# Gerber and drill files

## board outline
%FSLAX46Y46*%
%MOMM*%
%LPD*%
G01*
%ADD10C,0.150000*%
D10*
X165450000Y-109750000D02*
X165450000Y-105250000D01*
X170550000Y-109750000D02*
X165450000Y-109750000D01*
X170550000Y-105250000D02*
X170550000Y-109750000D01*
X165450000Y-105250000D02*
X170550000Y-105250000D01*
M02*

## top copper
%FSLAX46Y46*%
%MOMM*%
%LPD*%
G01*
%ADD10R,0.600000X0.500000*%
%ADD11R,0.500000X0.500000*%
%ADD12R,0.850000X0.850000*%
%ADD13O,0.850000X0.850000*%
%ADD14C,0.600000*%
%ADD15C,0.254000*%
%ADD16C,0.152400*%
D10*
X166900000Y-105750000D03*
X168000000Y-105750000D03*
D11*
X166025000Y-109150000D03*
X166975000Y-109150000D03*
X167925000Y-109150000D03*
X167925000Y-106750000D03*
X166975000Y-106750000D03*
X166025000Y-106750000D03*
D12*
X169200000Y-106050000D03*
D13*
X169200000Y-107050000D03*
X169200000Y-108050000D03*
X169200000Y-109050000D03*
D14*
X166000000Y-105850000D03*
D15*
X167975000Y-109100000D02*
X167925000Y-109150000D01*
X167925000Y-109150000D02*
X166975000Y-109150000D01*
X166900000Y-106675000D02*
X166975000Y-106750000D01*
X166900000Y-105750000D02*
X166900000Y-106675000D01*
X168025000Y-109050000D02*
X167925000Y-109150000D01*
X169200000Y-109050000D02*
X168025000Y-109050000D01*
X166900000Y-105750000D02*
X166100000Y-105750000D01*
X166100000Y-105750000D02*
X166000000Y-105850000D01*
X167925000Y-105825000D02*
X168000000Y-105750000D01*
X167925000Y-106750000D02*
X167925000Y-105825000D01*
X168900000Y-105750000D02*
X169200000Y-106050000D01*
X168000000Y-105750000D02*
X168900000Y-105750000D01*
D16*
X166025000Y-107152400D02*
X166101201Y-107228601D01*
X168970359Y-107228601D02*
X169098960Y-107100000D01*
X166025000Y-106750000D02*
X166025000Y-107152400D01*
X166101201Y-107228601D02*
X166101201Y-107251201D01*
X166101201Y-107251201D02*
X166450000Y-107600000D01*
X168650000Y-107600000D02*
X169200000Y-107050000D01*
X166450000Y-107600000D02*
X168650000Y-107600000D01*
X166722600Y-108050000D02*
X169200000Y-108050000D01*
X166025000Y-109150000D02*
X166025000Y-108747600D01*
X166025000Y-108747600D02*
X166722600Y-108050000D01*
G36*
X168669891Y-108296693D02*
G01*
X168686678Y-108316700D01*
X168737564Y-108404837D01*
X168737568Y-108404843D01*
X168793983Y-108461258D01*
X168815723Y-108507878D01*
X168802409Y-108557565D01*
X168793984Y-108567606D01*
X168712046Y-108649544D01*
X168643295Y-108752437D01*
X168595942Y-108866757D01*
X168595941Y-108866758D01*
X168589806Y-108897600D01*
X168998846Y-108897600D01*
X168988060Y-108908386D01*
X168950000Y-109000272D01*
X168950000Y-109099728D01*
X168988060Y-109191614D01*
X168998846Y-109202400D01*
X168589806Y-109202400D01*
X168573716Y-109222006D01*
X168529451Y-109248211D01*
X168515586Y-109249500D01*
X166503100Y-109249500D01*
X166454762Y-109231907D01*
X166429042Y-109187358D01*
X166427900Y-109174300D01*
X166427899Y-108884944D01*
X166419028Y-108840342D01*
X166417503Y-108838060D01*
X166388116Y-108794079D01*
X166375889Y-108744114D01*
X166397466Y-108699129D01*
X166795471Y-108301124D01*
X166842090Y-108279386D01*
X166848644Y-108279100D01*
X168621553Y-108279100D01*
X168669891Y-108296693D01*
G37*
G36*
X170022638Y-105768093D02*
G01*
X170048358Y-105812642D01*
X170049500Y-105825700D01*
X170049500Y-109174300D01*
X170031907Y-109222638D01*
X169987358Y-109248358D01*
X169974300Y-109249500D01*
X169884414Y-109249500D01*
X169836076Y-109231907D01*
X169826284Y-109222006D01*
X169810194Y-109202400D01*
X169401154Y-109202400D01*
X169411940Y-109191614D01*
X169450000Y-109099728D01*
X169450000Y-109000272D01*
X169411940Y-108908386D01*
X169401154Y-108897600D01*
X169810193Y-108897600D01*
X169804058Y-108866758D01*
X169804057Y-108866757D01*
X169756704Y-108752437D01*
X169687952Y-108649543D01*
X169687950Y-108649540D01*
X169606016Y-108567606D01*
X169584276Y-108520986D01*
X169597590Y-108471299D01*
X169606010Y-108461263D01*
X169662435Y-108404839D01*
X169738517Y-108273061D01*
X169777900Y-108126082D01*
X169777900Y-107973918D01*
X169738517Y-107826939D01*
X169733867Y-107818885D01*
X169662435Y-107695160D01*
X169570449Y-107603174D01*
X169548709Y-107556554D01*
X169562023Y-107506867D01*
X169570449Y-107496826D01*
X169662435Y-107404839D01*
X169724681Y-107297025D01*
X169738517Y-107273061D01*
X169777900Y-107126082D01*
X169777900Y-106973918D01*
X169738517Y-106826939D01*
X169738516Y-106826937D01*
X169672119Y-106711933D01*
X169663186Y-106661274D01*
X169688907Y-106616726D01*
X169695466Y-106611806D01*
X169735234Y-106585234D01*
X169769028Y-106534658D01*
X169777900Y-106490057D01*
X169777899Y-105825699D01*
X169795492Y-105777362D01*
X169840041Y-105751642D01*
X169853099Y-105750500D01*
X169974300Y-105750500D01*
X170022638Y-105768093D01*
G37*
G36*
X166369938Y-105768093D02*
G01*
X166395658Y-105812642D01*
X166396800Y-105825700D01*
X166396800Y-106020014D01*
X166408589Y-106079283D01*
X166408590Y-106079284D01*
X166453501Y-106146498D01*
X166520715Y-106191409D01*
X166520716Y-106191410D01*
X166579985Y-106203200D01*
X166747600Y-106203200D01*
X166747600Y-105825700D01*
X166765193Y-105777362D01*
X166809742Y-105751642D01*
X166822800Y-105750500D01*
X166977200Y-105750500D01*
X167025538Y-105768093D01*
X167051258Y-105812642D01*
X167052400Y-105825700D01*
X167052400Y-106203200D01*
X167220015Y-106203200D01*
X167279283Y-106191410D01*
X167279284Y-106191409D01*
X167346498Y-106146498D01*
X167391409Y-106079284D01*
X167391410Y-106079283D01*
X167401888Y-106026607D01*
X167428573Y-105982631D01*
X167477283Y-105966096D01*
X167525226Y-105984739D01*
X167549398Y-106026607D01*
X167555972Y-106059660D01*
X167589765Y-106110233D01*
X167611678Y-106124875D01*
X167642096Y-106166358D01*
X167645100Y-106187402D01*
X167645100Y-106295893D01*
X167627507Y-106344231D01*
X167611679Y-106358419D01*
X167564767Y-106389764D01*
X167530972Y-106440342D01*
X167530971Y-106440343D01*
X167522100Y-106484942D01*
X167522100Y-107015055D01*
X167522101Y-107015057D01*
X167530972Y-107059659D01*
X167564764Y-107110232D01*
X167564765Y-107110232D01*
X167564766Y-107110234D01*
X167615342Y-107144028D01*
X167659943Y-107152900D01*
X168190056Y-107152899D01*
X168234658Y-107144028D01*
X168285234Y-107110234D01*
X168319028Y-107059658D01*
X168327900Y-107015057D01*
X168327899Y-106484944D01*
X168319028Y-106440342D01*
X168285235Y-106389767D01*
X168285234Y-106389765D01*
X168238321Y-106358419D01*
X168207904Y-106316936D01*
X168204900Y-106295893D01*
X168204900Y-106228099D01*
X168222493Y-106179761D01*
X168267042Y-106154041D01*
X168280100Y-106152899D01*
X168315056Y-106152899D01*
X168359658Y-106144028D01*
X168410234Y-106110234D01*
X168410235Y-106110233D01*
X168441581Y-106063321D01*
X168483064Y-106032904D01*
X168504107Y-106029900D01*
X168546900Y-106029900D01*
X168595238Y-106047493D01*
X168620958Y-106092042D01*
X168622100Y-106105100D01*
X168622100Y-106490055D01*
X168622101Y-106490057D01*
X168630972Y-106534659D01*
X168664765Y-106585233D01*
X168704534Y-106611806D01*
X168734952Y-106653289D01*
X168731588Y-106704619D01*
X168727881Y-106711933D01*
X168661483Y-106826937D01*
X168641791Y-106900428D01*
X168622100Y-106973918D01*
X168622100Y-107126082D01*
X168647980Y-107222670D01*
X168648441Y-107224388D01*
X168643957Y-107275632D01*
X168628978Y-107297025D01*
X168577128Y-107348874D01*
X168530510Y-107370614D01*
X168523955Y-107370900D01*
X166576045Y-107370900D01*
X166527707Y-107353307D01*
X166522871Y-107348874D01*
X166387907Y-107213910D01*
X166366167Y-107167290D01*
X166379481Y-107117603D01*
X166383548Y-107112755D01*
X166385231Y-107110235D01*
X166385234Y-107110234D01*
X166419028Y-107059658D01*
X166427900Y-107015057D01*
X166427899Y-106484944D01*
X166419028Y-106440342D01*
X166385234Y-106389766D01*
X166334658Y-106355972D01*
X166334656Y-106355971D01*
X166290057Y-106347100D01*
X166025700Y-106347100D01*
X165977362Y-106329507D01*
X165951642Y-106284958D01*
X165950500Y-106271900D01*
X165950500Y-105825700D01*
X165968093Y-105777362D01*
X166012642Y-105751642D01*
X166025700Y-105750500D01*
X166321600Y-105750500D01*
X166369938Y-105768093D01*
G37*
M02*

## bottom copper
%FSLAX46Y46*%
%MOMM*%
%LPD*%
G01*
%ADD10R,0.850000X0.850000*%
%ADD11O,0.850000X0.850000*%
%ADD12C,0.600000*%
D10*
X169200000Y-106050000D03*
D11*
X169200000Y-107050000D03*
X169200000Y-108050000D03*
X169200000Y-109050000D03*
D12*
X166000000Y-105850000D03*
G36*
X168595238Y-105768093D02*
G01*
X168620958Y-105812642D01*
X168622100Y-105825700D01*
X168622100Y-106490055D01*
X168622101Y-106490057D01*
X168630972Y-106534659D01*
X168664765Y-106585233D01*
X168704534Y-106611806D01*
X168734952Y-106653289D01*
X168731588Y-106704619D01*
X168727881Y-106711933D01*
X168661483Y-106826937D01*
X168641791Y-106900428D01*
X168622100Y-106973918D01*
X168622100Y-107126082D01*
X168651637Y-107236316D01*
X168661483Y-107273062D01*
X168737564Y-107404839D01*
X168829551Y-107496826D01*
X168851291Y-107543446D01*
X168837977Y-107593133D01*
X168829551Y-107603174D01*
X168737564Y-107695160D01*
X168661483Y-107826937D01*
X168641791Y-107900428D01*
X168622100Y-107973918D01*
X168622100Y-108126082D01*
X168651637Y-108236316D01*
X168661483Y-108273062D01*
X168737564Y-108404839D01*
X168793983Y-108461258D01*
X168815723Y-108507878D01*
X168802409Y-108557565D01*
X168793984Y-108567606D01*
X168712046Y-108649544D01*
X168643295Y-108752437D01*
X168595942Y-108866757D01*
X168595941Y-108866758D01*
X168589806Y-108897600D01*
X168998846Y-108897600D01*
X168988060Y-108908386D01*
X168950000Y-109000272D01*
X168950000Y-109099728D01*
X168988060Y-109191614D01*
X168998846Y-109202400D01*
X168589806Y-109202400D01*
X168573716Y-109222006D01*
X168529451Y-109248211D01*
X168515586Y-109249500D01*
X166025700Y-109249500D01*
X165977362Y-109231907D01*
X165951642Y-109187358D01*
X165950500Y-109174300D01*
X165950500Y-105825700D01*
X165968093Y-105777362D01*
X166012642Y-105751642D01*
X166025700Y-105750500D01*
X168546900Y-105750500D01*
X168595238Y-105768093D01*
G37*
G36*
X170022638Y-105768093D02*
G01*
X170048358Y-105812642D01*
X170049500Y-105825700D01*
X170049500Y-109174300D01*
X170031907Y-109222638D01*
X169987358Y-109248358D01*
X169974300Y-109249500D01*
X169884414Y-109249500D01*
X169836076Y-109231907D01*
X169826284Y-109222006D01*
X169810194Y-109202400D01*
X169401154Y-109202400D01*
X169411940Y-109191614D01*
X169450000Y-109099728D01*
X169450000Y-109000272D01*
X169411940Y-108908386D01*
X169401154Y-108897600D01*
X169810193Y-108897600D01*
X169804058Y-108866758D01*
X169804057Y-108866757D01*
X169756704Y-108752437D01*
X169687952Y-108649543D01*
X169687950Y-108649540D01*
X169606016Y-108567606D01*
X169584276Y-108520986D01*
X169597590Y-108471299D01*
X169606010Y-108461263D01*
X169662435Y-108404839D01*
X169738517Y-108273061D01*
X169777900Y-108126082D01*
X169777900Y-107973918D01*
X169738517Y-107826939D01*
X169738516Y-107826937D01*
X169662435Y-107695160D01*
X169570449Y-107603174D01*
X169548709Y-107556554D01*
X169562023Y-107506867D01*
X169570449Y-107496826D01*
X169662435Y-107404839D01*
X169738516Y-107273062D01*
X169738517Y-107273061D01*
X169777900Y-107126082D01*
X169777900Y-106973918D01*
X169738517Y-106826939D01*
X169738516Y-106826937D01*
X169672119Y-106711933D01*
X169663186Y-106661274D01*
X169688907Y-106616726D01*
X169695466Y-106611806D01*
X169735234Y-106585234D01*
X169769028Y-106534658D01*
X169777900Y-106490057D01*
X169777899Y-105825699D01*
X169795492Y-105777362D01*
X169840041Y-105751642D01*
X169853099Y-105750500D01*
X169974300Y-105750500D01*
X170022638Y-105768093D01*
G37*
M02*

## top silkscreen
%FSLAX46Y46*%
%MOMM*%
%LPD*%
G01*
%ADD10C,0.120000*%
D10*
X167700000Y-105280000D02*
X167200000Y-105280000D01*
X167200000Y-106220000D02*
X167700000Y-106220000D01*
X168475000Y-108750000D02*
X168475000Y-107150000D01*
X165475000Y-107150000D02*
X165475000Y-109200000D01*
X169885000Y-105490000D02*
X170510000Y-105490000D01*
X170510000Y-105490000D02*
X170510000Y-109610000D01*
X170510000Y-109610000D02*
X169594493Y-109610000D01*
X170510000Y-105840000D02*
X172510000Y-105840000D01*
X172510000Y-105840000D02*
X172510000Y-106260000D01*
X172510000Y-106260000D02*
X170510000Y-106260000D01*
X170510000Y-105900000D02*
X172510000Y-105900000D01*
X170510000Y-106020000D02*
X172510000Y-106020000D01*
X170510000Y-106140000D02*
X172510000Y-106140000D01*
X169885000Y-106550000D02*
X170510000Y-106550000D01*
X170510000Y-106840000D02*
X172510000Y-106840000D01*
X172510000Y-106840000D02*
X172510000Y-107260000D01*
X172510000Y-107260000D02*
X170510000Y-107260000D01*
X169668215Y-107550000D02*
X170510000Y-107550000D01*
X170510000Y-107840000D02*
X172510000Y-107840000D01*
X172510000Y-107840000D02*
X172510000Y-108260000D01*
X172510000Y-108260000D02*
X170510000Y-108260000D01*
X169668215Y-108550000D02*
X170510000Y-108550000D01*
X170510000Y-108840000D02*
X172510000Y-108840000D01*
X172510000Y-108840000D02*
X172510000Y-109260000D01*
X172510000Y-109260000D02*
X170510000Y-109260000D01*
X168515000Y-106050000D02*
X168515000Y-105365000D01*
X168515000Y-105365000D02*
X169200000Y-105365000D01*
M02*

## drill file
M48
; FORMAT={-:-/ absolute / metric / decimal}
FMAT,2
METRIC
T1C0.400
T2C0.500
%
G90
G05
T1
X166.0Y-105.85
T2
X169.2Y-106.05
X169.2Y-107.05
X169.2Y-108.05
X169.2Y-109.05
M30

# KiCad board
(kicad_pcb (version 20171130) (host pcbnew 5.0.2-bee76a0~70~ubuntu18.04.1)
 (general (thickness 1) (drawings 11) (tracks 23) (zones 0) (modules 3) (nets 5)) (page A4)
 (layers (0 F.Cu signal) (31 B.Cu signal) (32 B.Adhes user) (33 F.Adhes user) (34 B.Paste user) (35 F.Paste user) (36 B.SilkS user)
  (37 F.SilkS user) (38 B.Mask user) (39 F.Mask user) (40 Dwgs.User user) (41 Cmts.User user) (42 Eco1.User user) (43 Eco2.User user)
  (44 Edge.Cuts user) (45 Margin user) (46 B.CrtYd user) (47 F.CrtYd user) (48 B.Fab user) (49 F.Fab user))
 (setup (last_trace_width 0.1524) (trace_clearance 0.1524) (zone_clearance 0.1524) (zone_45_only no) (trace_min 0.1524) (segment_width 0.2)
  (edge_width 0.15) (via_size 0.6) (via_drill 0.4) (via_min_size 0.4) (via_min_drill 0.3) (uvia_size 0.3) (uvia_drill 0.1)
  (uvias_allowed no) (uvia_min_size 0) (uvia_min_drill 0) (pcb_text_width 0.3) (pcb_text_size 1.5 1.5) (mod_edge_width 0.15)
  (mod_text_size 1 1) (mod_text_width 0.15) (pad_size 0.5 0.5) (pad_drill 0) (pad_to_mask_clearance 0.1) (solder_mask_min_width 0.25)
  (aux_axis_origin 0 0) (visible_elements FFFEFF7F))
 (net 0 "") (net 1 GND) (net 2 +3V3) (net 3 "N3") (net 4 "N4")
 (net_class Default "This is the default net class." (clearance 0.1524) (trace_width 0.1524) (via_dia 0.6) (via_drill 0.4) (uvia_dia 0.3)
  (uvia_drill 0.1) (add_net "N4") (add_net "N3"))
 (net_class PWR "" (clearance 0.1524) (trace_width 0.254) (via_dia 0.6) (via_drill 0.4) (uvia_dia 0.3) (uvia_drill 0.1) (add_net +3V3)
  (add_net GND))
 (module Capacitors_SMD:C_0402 (layer F.Cu) (at 167.45 105.75)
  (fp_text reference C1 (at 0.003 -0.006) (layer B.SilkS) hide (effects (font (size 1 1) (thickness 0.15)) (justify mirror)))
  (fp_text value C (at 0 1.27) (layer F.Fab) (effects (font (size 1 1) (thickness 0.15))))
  (fp_line (start 0.25 -0.47) (end -0.25 -0.47) (layer F.SilkS) (width 0.12))
  (fp_line (start -0.25 0.47) (end 0.25 0.47) (layer F.SilkS) (width 0.12))
  (pad 1 smd rect (at -0.55 0) (size 0.6 0.5) (layers F.Cu F.Paste F.Mask) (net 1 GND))
  (pad 2 smd rect (at 0.55 0) (size 0.6 0.5) (layers F.Cu F.Paste F.Mask) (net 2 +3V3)))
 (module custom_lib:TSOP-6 (layer F.Cu) (at 166.975 107.95 90)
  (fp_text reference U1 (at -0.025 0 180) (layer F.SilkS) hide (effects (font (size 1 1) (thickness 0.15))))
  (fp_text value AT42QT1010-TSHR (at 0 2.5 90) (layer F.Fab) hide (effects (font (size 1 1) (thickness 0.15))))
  (fp_line (start -0.8 1.5) (end 0.8 1.5) (layer F.SilkS) (width 0.12))
  (fp_line (start 0.8 -1.5) (end -1.25 -1.5) (layer F.SilkS) (width 0.12))
  (pad 1 smd rect (at -1.2 -0.95 90) (size 0.5 0.5) (layers F.Cu F.Paste F.Mask) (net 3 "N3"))
  (pad 2 smd rect (at -1.2 0 90) (size 0.5 0.5) (layers F.Cu F.Paste F.Mask) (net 1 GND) (zone_connect 2))
  (pad 3 smd rect (at -1.2 0.95 90) (size 0.5 0.5) (layers F.Cu F.Paste F.Mask) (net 1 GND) (zone_connect 2))
  (pad 4 smd rect (at 1.2 0.95 90) (size 0.5 0.5) (layers F.Cu F.Paste F.Mask) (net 2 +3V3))
  (pad 5 smd rect (at 1.2 0 90) (size 0.5 0.5) (layers F.Cu F.Paste F.Mask) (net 1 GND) (zone_connect 2))
  (pad 6 smd rect (at 1.2 -0.95 90) (size 0.5 0.5) (layers F.Cu F.Paste F.Mask) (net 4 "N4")))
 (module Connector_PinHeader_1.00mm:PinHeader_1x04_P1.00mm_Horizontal (layer F.Cu) (at 169.2 106.05)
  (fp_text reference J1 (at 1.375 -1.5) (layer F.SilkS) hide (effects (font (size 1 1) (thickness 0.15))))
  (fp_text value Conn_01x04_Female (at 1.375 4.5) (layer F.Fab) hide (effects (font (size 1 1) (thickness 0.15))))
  (fp_line (start 0.685 -0.56) (end 1.31 -0.56) (layer F.SilkS) (width 0.12))
  (fp_line (start 1.31 -0.56) (end 1.31 3.56) (layer F.SilkS) (width 0.12))
  (fp_line (start 1.31 3.56) (end 0.394493 3.56) (layer F.SilkS) (width 0.12))
  (fp_line (start 1.31 -0.21) (end 3.31 -0.21) (layer F.SilkS) (width 0.12))
  (fp_line (start 3.31 -0.21) (end 3.31 0.21) (layer F.SilkS) (width 0.12))
  (fp_line (start 3.31 0.21) (end 1.31 0.21) (layer F.SilkS) (width 0.12))
  (fp_line (start 1.31 -0.15) (end 3.31 -0.15) (layer F.SilkS) (width 0.12))
  (fp_line (start 1.31 -0.03) (end 3.31 -0.03) (layer F.SilkS) (width 0.12))
  (fp_line (start 1.31 0.09) (end 3.31 0.09) (layer F.SilkS) (width 0.12))
  (fp_line (start 0.685 0.5) (end 1.31 0.5) (layer F.SilkS) (width 0.12))
  (fp_line (start 1.31 0.79) (end 3.31 0.79) (layer F.SilkS) (width 0.12))
  (fp_line (start 3.31 0.79) (end 3.31 1.21) (layer F.SilkS) (width 0.12))
  (fp_line (start 3.31 1.21) (end 1.31 1.21) (layer F.SilkS) (width 0.12))
  (fp_line (start 0.468215 1.5) (end 1.31 1.5) (layer F.SilkS) (width 0.12))
  (fp_line (start 1.31 1.79) (end 3.31 1.79) (layer F.SilkS) (width 0.12))
  (fp_line (start 3.31 1.79) (end 3.31 2.21) (layer F.SilkS) (width 0.12))
  (fp_line (start 3.31 2.21) (end 1.31 2.21) (layer F.SilkS) (width 0.12))
  (fp_line (start 0.468215 2.5) (end 1.31 2.5) (layer F.SilkS) (width 0.12))
  (fp_line (start 1.31 2.79) (end 3.31 2.79) (layer F.SilkS) (width 0.12))
  (fp_line (start 3.31 2.79) (end 3.31 3.21) (layer F.SilkS) (width 0.12))
  (fp_line (start 3.31 3.21) (end 1.31 3.21) (layer F.SilkS) (width 0.12))
  (fp_line (start -0.685 0) (end -0.685 -0.685) (layer F.SilkS) (width 0.12))
  (fp_line (start -0.685 -0.685) (end 0 -0.685) (layer F.SilkS) (width 0.12))
  (pad 1 thru_hole rect (at 0 0) (size 0.85 0.85) (drill 0.5) (layers *.Cu *.Mask) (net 2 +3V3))
  (pad 2 thru_hole oval (at 0 1) (size 0.85 0.85) (drill 0.5) (layers *.Cu *.Mask) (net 4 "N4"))
  (pad 3 thru_hole oval (at 0 2) (size 0.85 0.85) (drill 0.5) (layers *.Cu *.Mask) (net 3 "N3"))
  (pad 4 thru_hole oval (at 0 3) (size 0.85 0.85) (drill 0.5) (layers *.Cu *.Mask) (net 1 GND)))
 (gr_line (start 165.45 109.75) (end 165.45 105.25) (layer Edge.Cuts) (width 0.15))
 (gr_line (start 170.55 109.75) (end 165.45 109.75) (layer Edge.Cuts) (width 0.15))
 (gr_line (start 170.55 105.25) (end 170.55 109.75) (layer Edge.Cuts) (width 0.15))
 (gr_line (start 165.45 105.25) (end 170.55 105.25) (layer Edge.Cuts) (width 0.15))
 (segment (start 167.975 109.1) (end 167.925 109.15) (width 0.254) (layer F.Cu) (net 1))
 (segment (start 167.925 109.15) (end 166.975 109.15) (width 0.254) (layer F.Cu) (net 1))
 (segment (start 166.9 106.675) (end 166.975 106.75) (width 0.254) (layer F.Cu) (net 1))
 (segment (start 166.9 105.75) (end 166.9 106.675) (width 0.254) (layer F.Cu) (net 1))
 (segment (start 168.025 109.05) (end 167.925 109.15) (width 0.254) (layer F.Cu) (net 1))
 (segment (start 169.2 109.05) (end 168.025 109.05) (width 0.254) (layer F.Cu) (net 1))
 (segment (start 166.9 105.75) (end 166.1 105.75) (width 0.254) (layer F.Cu) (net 1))
 (via (at 166 105.85) (size 0.6) (drill 0.4) (layers F.Cu B.Cu) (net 1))
 (segment (start 166.1 105.75) (end 166 105.85) (width 0.254) (layer F.Cu) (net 1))
 (segment (start 167.925 105.825) (end 168 105.75) (width 0.254) (layer F.Cu) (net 2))
 (segment (start 167.925 106.75) (end 167.925 105.825) (width 0.254) (layer F.Cu) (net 2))
 (segment (start 168.9 105.75) (end 169.2 106.05) (width 0.254) (layer F.Cu) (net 2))
 (segment (start 168 105.75) (end 168.9 105.75) (width 0.254) (layer F.Cu) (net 2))
 (segment (start 166.025 107.1524) (end 166.101201 107.228601) (width 0.1524) (layer F.Cu) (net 4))
 (segment (start 168.970359 107.228601) (end 169.09896 107.1) (width 0.1524) (layer F.Cu) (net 4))
 (segment (start 166.025 106.75) (end 166.025 107.1524) (width 0.1524) (layer F.Cu) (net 4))
 (segment (start 166.101201 107.228601) (end 166.101201 107.251201) (width 0.1524) (layer F.Cu) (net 4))
 (segment (start 166.101201 107.251201) (end 166.45 107.6) (width 0.1524) (layer F.Cu) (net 4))
 (segment (start 168.65 107.6) (end 169.2 107.05) (width 0.1524) (layer F.Cu) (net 4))
 (segment (start 166.45 107.6) (end 168.65 107.6) (width 0.1524) (layer F.Cu) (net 4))
 (segment (start 166.7226 108.05) (end 169.2 108.05) (width 0.1524) (layer F.Cu) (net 3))
 (segment (start 166.025 109.15) (end 166.025 108.7476) (width 0.1524) (layer F.Cu) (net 3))
 (segment (start 166.025 108.7476) (end 166.7226 108.05) (width 0.1524) (layer F.Cu) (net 3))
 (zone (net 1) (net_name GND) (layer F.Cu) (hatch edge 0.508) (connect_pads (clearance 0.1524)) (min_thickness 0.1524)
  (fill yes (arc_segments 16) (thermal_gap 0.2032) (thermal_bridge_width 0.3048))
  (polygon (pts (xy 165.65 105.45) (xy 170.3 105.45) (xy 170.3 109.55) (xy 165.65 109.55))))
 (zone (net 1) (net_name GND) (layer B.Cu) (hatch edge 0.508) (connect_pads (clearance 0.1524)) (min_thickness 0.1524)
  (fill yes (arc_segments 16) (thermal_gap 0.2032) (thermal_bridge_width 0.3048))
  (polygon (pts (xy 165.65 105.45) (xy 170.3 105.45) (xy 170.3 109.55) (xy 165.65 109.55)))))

